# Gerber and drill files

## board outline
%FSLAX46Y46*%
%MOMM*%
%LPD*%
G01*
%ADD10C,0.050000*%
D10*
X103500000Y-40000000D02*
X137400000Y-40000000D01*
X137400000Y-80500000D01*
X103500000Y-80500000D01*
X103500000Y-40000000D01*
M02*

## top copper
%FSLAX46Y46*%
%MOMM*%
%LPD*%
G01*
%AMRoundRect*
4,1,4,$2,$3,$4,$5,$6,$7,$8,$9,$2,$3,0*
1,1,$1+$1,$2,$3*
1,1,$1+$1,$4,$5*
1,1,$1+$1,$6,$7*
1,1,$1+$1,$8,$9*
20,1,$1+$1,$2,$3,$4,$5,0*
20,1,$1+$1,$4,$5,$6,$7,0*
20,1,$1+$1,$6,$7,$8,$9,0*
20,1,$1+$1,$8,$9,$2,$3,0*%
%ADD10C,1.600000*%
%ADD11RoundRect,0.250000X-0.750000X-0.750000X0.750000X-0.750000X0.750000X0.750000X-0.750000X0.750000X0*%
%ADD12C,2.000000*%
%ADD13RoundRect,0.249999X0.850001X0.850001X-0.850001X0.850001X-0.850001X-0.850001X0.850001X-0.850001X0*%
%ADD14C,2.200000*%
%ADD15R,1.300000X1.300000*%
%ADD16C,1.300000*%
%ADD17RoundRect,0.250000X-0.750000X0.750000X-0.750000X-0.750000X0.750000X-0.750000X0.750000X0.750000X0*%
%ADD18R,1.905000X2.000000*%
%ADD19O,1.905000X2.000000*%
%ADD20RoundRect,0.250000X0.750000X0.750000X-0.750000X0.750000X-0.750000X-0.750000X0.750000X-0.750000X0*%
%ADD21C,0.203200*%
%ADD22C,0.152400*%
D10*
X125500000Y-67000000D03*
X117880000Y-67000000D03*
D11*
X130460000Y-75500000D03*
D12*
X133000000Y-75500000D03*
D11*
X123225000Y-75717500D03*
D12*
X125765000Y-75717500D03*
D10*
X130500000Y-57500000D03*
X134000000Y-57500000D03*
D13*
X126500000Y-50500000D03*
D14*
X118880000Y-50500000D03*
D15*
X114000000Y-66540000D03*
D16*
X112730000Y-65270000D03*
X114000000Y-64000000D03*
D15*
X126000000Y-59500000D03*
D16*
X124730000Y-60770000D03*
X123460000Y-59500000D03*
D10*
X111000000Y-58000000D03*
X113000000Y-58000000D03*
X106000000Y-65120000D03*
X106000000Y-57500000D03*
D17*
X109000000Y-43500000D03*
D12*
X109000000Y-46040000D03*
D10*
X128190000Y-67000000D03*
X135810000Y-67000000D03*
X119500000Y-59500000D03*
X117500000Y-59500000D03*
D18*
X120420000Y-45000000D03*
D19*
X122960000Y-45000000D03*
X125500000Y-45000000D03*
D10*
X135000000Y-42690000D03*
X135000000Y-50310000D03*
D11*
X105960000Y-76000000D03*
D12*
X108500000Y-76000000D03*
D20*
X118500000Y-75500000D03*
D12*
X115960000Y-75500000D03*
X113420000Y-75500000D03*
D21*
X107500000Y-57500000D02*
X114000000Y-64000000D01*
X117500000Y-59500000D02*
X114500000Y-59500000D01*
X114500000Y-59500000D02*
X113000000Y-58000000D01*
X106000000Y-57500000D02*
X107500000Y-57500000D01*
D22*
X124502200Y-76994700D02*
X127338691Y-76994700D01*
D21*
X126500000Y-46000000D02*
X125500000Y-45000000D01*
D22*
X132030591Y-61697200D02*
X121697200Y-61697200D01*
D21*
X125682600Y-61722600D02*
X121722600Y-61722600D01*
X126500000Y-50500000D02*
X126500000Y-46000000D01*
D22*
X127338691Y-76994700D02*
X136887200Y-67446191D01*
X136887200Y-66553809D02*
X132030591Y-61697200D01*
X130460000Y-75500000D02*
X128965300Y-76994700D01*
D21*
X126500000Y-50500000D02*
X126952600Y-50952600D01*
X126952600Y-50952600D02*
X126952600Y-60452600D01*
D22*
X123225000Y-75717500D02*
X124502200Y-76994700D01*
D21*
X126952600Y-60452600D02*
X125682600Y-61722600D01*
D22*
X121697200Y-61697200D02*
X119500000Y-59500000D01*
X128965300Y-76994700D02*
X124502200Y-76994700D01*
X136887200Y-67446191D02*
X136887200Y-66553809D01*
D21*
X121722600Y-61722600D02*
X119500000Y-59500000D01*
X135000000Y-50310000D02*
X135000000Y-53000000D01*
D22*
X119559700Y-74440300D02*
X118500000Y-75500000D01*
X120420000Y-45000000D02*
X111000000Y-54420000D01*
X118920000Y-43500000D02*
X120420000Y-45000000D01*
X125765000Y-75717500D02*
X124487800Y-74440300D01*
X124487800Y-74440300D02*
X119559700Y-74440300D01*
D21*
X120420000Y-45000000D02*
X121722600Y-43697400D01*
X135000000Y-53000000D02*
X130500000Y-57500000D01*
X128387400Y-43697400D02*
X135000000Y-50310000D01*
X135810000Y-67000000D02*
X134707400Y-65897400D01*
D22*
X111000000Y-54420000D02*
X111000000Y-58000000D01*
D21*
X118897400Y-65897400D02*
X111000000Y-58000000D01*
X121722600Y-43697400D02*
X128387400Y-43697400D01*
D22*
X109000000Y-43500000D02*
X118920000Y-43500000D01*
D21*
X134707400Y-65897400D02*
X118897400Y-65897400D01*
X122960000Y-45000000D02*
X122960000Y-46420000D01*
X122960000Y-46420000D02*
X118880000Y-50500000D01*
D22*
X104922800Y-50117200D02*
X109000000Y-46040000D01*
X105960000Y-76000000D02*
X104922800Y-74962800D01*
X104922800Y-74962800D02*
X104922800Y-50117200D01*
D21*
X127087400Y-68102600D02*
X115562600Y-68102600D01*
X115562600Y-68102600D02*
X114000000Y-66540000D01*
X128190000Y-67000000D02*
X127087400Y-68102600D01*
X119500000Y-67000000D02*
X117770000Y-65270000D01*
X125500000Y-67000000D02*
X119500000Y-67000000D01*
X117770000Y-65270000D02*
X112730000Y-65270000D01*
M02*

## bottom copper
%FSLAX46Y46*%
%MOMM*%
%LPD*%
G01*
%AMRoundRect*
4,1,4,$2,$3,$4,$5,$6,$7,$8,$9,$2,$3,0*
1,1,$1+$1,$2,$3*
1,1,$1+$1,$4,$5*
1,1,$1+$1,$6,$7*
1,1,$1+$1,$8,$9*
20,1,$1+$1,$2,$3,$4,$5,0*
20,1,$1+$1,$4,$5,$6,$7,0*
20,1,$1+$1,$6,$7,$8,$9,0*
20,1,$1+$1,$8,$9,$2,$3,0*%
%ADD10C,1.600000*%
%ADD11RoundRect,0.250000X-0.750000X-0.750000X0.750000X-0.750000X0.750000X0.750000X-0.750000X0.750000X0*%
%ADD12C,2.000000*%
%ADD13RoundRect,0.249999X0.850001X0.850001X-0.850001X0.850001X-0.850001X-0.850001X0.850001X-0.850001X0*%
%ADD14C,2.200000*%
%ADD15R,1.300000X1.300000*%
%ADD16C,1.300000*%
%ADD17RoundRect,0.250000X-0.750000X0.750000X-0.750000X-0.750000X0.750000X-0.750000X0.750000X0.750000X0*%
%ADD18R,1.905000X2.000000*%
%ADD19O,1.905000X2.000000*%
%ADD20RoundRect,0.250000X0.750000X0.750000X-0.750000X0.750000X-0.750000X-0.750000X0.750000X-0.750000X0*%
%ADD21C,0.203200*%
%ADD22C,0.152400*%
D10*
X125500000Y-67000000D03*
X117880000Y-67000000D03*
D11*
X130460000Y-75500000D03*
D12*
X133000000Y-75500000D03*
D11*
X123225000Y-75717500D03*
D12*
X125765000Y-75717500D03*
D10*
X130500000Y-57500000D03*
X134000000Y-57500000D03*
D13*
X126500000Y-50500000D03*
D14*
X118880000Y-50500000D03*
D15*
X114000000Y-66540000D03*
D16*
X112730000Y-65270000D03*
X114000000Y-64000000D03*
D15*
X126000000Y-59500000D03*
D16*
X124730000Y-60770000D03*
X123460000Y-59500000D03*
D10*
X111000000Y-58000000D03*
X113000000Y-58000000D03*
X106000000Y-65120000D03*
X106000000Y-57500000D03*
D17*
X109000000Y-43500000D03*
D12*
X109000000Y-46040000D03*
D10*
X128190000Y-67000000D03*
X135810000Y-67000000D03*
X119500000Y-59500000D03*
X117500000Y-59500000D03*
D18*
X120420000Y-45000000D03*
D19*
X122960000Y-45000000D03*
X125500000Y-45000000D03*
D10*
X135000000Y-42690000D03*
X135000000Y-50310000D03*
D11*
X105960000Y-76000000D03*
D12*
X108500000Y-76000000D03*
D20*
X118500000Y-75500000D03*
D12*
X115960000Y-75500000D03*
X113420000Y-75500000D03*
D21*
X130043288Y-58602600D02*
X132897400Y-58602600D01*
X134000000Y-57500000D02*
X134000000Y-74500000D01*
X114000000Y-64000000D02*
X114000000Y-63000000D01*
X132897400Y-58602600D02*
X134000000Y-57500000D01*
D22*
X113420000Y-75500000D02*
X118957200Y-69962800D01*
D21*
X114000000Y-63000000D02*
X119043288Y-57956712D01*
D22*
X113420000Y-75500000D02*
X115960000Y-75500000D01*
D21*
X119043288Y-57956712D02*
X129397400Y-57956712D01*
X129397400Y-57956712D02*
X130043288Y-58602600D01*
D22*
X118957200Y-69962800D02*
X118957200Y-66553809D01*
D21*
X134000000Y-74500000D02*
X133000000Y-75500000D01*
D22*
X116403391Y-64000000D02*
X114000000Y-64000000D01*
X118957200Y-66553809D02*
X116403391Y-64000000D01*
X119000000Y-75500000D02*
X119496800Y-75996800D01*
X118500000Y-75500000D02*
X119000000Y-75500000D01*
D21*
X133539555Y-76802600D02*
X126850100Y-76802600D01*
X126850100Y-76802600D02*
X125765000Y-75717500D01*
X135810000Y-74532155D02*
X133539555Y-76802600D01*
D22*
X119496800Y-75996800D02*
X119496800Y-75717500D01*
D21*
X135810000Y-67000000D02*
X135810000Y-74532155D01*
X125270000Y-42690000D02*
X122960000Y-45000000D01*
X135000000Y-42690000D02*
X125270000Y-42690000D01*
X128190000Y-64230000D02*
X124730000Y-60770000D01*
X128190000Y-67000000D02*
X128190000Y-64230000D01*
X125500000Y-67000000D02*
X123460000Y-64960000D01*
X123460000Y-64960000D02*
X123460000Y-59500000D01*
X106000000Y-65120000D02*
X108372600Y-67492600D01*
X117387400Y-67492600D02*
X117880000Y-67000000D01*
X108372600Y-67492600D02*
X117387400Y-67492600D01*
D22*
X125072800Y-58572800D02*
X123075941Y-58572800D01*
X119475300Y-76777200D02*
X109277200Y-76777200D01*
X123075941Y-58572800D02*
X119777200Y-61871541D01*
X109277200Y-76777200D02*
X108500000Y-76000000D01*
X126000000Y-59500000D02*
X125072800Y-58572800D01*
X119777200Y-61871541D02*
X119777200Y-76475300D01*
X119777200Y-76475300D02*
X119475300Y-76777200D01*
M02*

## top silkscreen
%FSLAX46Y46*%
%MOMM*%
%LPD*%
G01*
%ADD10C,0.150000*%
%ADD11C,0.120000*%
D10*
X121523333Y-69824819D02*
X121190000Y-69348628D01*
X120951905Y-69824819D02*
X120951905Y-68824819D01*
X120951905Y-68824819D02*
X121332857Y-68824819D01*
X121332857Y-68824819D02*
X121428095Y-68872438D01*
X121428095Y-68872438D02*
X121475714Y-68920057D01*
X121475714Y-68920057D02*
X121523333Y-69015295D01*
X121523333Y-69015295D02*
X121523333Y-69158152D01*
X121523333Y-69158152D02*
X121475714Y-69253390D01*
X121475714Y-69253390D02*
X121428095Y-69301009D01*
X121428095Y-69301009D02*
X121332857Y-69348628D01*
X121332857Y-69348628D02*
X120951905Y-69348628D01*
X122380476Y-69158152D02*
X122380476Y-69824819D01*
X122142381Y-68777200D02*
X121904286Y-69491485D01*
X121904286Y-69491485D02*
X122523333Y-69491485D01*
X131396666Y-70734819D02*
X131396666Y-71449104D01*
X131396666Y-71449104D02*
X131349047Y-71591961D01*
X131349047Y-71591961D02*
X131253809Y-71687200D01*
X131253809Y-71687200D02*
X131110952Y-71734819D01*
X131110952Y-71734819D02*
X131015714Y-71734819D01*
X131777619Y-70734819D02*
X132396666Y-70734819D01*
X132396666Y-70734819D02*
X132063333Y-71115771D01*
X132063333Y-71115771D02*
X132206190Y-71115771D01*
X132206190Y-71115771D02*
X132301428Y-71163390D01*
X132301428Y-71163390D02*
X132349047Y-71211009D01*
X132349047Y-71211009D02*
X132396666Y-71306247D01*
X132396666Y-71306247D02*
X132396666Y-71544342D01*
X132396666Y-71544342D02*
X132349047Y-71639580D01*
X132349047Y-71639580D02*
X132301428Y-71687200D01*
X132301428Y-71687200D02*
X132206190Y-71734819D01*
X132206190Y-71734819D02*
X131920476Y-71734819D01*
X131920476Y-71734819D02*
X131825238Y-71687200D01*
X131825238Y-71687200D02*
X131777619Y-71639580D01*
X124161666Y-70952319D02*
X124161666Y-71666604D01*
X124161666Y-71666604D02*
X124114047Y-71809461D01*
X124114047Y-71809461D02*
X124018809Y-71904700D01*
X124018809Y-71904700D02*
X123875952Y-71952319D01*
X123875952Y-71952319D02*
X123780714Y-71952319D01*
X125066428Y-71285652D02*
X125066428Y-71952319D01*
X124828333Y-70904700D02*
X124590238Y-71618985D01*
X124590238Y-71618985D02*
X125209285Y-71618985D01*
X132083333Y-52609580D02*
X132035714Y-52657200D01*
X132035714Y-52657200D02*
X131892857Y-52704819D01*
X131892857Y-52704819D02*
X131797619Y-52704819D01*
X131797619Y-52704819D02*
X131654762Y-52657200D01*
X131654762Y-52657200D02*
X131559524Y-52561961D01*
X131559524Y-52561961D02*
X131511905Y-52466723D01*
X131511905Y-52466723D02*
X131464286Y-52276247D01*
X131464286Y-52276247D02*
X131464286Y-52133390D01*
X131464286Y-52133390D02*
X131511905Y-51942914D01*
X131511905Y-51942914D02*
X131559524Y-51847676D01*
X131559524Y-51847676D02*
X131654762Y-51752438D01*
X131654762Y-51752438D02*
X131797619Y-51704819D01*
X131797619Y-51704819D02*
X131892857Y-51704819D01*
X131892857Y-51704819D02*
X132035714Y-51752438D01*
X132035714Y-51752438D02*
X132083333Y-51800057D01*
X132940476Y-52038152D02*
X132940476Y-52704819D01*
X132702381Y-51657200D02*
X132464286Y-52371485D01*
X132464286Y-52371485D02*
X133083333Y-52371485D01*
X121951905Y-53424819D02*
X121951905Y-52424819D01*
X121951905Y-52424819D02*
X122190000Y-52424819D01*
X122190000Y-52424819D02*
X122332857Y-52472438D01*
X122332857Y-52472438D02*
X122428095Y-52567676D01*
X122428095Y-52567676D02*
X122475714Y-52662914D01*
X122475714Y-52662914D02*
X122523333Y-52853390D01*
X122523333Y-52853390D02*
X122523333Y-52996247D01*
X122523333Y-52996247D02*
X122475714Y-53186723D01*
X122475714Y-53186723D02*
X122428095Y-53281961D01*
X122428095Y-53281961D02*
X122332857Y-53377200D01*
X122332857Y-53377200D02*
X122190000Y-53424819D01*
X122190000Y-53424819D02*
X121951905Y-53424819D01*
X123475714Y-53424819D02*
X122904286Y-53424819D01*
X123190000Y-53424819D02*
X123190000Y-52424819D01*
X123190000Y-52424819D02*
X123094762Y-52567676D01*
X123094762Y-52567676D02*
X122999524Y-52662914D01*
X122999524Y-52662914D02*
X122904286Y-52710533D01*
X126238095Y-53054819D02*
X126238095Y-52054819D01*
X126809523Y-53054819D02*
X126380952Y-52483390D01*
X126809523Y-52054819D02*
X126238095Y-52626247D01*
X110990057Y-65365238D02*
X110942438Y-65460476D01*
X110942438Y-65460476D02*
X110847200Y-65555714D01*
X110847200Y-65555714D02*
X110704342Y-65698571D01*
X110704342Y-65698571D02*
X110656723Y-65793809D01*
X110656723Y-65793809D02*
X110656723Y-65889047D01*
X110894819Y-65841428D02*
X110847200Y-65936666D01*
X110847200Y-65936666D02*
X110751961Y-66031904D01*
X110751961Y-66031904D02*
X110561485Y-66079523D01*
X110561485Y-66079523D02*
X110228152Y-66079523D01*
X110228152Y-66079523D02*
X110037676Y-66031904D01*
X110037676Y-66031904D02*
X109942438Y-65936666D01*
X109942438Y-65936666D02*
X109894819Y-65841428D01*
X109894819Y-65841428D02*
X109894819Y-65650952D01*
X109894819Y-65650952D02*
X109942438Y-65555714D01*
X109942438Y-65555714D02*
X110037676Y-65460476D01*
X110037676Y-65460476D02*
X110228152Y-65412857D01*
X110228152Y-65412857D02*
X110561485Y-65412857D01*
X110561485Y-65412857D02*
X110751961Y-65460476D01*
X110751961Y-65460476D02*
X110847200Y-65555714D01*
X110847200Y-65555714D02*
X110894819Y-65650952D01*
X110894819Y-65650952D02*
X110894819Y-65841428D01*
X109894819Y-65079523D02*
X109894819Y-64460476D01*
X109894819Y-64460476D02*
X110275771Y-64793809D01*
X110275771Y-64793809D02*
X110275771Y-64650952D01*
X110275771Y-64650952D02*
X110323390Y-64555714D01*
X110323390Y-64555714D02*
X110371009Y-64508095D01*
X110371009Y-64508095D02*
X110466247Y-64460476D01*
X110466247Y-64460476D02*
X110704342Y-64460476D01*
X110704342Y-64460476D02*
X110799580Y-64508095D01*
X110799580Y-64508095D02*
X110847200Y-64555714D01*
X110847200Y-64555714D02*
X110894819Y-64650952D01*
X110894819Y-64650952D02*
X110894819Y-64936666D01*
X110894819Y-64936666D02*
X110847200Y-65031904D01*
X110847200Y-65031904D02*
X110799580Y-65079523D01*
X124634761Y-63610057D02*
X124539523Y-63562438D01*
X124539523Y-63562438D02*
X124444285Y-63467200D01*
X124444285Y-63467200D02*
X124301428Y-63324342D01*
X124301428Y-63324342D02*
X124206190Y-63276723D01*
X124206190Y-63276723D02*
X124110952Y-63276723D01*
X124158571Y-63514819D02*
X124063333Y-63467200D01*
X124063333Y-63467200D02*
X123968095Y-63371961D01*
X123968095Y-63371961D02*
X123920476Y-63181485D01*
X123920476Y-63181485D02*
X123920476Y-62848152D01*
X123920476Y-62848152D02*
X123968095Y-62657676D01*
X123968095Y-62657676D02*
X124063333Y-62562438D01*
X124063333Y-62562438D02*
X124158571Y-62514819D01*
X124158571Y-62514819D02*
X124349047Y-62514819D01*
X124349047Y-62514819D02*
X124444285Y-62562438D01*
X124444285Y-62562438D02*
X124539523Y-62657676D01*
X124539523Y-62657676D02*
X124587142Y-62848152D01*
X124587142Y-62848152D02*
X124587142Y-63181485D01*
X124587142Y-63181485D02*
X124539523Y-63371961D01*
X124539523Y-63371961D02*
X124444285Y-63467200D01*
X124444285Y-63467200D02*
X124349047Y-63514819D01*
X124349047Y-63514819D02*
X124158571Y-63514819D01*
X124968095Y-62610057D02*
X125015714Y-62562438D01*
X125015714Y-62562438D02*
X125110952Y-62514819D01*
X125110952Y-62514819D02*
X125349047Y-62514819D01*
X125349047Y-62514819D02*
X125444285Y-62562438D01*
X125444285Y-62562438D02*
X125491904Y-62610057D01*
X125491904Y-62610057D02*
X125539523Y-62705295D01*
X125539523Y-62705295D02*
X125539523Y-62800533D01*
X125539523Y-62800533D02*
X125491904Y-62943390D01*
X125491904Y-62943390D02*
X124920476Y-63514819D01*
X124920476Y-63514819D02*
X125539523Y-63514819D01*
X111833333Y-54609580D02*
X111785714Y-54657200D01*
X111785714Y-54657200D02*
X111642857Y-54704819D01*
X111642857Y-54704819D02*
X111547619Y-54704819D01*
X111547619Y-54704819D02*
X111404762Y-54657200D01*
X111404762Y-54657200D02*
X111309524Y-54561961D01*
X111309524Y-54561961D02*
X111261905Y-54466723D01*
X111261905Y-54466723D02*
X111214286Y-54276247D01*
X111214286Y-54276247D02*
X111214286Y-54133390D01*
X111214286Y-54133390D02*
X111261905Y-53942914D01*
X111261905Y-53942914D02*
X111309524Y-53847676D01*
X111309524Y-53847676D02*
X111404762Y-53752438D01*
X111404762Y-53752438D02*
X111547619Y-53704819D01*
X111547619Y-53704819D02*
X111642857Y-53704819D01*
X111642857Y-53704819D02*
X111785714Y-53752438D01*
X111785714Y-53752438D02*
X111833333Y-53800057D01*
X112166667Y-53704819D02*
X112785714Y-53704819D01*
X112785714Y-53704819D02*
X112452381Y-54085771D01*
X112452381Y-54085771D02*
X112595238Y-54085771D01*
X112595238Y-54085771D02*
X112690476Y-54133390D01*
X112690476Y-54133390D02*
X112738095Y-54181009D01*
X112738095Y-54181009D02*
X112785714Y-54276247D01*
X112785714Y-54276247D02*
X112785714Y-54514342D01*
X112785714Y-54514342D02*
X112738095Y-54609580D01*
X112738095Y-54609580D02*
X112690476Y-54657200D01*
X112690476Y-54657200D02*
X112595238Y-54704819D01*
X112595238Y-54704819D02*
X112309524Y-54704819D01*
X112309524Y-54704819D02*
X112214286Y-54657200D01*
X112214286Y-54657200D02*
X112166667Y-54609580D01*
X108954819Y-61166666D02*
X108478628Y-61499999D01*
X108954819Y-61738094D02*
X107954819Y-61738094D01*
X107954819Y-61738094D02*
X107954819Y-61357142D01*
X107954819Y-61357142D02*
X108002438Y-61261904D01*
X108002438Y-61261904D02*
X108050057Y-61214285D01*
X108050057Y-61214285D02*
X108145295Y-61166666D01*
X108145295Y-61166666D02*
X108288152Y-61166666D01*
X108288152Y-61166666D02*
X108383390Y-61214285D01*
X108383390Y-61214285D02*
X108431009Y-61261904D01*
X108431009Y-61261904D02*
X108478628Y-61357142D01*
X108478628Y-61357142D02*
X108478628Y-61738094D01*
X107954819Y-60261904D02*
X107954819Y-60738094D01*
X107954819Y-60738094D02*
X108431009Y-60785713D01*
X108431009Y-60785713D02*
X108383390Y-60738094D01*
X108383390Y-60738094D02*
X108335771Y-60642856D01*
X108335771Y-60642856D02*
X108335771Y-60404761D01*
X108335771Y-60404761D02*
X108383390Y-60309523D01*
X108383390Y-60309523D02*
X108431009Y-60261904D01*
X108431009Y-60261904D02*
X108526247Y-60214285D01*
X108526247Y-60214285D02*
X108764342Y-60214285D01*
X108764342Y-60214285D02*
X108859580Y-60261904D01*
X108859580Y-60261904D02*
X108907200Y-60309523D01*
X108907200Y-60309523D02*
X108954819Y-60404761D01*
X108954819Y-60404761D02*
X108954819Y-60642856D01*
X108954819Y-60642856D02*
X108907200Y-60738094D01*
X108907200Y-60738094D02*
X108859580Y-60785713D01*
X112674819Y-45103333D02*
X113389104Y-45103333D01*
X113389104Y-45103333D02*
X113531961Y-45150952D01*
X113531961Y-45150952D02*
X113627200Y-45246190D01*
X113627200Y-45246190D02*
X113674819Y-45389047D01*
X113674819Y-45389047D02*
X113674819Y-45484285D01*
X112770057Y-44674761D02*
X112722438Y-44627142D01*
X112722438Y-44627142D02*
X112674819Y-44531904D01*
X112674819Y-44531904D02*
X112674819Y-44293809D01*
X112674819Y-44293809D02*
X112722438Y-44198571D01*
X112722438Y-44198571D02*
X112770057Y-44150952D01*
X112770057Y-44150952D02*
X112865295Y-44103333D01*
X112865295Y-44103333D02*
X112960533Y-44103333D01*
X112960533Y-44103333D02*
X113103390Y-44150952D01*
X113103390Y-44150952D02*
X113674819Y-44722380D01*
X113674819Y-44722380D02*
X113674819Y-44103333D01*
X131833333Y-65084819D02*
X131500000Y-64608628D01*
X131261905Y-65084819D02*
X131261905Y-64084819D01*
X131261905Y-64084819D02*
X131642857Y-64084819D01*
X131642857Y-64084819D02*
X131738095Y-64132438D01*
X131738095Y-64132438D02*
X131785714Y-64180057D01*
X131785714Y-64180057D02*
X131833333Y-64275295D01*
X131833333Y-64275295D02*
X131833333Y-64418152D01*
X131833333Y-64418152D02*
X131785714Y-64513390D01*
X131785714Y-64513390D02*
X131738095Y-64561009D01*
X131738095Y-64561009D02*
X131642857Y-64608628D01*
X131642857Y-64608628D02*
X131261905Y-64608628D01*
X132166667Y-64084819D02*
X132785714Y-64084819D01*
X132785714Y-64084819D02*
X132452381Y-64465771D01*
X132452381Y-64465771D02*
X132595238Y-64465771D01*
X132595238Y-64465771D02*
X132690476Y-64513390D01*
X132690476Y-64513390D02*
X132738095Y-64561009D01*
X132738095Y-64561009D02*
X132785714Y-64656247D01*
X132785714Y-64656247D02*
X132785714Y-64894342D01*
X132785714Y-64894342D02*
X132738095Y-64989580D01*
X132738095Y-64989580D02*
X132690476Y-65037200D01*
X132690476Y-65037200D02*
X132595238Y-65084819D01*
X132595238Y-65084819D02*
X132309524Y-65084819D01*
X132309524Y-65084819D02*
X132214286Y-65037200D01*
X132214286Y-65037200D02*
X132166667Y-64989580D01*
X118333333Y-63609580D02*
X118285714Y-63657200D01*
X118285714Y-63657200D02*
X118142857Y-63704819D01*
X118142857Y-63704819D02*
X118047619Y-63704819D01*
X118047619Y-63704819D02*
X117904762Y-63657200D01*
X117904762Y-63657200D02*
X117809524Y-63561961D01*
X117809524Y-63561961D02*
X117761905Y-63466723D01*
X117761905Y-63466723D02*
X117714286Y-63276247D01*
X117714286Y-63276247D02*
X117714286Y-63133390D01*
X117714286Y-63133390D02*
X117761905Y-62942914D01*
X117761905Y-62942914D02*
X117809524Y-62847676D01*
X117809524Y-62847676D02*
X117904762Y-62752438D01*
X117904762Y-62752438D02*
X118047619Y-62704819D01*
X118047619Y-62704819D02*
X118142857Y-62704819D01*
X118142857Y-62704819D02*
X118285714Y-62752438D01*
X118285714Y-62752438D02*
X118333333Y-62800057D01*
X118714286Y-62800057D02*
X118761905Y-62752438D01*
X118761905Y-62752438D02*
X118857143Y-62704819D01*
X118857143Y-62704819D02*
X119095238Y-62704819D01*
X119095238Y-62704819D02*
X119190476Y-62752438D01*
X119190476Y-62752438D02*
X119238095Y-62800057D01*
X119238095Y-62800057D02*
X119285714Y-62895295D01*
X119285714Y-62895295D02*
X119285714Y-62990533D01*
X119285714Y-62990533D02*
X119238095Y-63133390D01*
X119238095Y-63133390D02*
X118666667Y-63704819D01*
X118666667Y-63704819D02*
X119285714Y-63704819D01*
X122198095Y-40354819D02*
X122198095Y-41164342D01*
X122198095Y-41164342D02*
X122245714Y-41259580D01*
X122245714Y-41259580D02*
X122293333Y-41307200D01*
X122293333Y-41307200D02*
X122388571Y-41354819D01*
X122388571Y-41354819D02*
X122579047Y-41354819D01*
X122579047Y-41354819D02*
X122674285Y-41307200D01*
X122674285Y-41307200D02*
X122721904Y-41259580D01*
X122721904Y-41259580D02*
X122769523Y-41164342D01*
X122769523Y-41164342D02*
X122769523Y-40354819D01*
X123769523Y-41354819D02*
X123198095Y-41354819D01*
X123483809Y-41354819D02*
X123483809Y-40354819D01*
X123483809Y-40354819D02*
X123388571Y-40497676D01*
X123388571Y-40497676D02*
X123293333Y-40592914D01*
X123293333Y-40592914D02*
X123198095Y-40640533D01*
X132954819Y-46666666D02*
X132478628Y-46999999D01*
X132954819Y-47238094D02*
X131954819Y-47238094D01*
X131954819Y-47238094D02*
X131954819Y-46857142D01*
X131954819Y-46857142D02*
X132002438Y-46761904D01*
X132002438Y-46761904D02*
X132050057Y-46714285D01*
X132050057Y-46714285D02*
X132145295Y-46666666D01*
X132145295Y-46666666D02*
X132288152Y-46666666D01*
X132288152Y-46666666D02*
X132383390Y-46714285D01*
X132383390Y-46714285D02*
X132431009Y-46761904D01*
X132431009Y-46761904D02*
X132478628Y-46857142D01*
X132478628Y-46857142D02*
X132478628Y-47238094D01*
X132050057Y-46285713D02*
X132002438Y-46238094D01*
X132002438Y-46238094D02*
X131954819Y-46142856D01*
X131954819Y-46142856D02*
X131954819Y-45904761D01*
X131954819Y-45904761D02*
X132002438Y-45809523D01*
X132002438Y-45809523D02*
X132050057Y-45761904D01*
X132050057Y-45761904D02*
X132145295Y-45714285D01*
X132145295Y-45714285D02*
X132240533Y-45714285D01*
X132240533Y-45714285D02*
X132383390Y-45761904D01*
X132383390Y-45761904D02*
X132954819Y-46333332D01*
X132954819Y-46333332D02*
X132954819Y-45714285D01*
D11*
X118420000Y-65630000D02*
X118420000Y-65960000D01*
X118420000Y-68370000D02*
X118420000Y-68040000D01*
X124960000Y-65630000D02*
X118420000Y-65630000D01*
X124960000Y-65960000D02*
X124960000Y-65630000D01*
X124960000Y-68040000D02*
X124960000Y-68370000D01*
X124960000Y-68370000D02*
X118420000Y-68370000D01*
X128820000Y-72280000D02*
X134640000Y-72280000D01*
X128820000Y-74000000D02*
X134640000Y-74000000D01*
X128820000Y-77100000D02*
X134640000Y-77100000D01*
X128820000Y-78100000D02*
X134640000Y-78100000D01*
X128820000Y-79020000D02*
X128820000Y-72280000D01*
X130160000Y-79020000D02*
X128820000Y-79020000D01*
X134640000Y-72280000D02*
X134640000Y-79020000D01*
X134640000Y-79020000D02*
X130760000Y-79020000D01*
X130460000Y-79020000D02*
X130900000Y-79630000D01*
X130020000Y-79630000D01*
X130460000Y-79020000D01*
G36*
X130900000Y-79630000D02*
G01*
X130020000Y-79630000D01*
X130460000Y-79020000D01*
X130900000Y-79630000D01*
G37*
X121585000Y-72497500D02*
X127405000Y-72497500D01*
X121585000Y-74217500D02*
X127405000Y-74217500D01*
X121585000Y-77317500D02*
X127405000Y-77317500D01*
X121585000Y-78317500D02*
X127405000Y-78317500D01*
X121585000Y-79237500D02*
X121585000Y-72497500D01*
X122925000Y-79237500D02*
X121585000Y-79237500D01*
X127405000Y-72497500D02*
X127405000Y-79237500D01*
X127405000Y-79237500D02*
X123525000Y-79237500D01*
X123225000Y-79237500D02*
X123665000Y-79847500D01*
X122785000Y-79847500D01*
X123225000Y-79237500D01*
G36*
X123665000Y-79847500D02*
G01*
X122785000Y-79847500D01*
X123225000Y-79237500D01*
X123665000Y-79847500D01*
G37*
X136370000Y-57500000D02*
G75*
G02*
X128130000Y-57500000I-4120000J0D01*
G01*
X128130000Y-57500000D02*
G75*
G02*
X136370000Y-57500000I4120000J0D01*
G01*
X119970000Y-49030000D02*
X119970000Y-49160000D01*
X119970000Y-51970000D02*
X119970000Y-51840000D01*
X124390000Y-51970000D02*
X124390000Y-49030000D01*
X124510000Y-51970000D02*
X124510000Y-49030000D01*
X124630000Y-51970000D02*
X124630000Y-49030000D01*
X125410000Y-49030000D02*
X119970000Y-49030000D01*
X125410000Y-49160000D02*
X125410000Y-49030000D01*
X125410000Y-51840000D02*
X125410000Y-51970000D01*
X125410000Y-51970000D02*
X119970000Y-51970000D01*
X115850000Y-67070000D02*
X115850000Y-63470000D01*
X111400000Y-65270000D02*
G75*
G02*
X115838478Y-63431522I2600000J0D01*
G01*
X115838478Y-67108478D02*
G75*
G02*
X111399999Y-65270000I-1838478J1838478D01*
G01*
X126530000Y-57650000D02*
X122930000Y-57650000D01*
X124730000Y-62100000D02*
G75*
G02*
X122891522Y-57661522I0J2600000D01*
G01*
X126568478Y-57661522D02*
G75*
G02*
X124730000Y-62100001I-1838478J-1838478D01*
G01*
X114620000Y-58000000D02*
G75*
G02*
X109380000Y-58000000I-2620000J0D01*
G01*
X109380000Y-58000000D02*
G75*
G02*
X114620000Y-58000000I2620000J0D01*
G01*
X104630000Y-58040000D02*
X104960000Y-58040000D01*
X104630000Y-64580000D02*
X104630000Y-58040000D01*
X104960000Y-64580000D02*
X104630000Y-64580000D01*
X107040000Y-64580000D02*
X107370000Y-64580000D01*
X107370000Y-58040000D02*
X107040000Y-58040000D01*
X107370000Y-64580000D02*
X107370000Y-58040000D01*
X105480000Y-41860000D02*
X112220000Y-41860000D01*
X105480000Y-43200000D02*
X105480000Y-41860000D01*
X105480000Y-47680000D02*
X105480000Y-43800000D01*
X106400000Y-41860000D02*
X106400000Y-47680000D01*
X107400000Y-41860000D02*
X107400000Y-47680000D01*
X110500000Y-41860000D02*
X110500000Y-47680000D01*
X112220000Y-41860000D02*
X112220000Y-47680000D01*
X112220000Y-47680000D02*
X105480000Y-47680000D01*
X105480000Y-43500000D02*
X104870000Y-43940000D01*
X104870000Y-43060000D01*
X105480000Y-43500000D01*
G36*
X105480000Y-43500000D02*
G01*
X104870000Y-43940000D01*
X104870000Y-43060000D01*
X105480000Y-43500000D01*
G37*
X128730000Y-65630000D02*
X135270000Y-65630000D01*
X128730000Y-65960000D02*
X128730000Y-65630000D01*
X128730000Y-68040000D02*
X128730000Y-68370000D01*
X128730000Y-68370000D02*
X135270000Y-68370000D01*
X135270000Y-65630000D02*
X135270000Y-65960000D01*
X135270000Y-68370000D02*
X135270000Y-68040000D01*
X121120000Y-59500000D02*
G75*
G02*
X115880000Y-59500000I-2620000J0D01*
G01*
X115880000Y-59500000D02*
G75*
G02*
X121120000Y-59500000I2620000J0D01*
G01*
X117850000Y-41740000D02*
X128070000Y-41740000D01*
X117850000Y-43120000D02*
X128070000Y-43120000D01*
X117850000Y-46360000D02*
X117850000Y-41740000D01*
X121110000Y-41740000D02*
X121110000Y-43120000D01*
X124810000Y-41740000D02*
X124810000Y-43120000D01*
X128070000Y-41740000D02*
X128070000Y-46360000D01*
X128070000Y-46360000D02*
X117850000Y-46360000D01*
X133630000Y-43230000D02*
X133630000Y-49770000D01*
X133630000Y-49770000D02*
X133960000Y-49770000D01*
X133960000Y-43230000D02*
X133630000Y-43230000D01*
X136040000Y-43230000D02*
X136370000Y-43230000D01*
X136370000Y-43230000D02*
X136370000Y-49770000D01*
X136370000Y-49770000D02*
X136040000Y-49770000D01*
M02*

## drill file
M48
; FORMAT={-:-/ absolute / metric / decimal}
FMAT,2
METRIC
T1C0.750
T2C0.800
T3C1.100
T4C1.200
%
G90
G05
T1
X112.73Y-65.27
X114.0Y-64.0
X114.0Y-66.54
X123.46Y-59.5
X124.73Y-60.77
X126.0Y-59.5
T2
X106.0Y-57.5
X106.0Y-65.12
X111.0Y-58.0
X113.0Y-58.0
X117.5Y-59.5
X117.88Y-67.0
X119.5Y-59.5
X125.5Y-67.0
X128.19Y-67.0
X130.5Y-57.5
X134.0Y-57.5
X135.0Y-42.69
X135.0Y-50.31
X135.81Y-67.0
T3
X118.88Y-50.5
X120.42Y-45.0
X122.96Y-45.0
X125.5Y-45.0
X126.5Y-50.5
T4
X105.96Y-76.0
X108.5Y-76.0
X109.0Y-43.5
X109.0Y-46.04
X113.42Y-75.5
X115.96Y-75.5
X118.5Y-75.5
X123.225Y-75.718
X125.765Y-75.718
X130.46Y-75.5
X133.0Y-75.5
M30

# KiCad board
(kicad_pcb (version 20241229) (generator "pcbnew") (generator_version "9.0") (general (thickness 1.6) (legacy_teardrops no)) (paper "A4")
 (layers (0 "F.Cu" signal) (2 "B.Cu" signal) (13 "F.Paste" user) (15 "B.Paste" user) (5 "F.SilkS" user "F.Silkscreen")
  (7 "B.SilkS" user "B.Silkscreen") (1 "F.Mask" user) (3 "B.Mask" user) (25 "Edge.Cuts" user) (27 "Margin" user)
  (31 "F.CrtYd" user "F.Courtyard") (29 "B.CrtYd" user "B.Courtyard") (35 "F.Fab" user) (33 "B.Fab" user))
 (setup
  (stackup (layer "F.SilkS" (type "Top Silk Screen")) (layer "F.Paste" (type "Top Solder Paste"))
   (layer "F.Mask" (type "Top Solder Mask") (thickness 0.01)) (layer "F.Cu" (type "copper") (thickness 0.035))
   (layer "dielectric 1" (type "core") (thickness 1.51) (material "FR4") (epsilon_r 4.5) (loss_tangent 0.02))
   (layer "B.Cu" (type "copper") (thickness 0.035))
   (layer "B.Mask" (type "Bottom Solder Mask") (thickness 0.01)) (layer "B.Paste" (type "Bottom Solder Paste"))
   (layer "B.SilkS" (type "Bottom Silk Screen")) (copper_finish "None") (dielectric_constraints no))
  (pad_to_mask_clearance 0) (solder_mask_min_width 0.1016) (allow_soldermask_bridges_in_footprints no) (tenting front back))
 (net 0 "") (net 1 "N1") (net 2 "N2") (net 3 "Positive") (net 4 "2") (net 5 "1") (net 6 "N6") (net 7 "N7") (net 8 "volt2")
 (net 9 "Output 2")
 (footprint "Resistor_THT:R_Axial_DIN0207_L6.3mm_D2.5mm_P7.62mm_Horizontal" (layer "F.Cu") (at 125.5 67 180)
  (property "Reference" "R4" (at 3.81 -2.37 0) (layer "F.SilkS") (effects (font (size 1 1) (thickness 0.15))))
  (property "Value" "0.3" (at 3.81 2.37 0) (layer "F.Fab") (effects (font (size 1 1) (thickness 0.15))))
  (fp_line (start 7.08 1.37) (end 7.08 1.04) (stroke (width 0.12) (type solid)) (layer "F.SilkS"))
  (fp_line (start 7.08 -1.37) (end 7.08 -1.04) (stroke (width 0.12) (type solid)) (layer "F.SilkS"))
  (fp_line (start 0.54 1.37) (end 7.08 1.37) (stroke (width 0.12) (type solid)) (layer "F.SilkS"))
  (fp_line (start 0.54 1.04) (end 0.54 1.37) (stroke (width 0.12) (type solid)) (layer "F.SilkS"))
  (fp_line (start 0.54 -1.04) (end 0.54 -1.37) (stroke (width 0.12) (type solid)) (layer "F.SilkS"))
  (fp_line (start 0.54 -1.37) (end 7.08 -1.37) (stroke (width 0.12) (type solid)) (layer "F.SilkS"))
  (pad "1" thru_hole circle (at 0 0 180) (size 1.6 1.6) (drill 0.8) (layers "*.Cu" "*.Mask") (remove_unused_layers no) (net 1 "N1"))
  (pad "2" thru_hole circle (at 7.62 0 180) (size 1.6 1.6) (drill 0.8) (layers "*.Cu" "*.Mask") (remove_unused_layers no) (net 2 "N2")))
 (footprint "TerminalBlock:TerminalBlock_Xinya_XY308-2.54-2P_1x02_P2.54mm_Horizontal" (layer "F.Cu") (at 130.46 75.5)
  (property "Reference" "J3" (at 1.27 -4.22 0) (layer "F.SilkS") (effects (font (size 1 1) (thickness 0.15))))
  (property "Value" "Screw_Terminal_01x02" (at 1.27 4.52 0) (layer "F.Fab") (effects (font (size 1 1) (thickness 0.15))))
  (fp_line (start -1.64 -3.22) (end 4.18 -3.22) (stroke (width 0.12) (type solid)) (layer "F.SilkS"))
  (fp_line (start -1.64 -1.5) (end 4.18 -1.5) (stroke (width 0.12) (type solid)) (layer "F.SilkS"))
  (fp_line (start -1.64 1.6) (end 4.18 1.6) (stroke (width 0.12) (type solid)) (layer "F.SilkS"))
  (fp_line (start -1.64 2.6) (end 4.18 2.6) (stroke (width 0.12) (type solid)) (layer "F.SilkS"))
  (fp_line (start -1.64 3.52) (end -1.64 -3.22) (stroke (width 0.12) (type solid)) (layer "F.SilkS"))
  (fp_line (start -0.3 3.52) (end -1.64 3.52) (stroke (width 0.12) (type solid)) (layer "F.SilkS"))
  (fp_line (start 4.18 -3.22) (end 4.18 3.52) (stroke (width 0.12) (type solid)) (layer "F.SilkS"))
  (fp_line (start 4.18 3.52) (end 0.3 3.52) (stroke (width 0.12) (type solid)) (layer "F.SilkS"))
  (fp_poly (pts (xy 0 3.52) (xy 0.44 4.13) (xy -0.44 4.13)) (stroke (width 0.12) (type solid)) (fill yes) (layer "F.SilkS"))
  (pad "1" thru_hole roundrect (at 0 0) (size 2 2) (drill 1.2) (layers "*.Cu" "*.Mask") (remove_unused_layers no) (roundrect_rratio 0.125)
   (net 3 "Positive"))
  (pad "2" thru_hole circle (at 2.54 0) (size 2 2) (drill 1.2) (layers "*.Cu" "*.Mask") (remove_unused_layers no) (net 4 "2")))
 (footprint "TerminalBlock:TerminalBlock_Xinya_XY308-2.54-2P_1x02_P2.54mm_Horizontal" (layer "F.Cu") (at 123.225 75.7175)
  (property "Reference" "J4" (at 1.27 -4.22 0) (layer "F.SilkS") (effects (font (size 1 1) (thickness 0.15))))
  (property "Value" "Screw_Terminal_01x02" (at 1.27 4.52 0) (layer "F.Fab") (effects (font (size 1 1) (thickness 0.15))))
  (fp_line (start -1.64 -3.22) (end 4.18 -3.22) (stroke (width 0.12) (type solid)) (layer "F.SilkS"))
  (fp_line (start -1.64 -1.5) (end 4.18 -1.5) (stroke (width 0.12) (type solid)) (layer "F.SilkS"))
  (fp_line (start -1.64 1.6) (end 4.18 1.6) (stroke (width 0.12) (type solid)) (layer "F.SilkS"))
  (fp_line (start -1.64 2.6) (end 4.18 2.6) (stroke (width 0.12) (type solid)) (layer "F.SilkS"))
  (fp_line (start -1.64 3.52) (end -1.64 -3.22) (stroke (width 0.12) (type solid)) (layer "F.SilkS"))
  (fp_line (start -0.3 3.52) (end -1.64 3.52) (stroke (width 0.12) (type solid)) (layer "F.SilkS"))
  (fp_line (start 4.18 -3.22) (end 4.18 3.52) (stroke (width 0.12) (type solid)) (layer "F.SilkS"))
  (fp_line (start 4.18 3.52) (end 0.3 3.52) (stroke (width 0.12) (type solid)) (layer "F.SilkS"))
  (fp_poly (pts (xy 0 3.52) (xy 0.44 4.13) (xy -0.44 4.13)) (stroke (width 0.12) (type solid)) (fill yes) (layer "F.SilkS"))
  (pad "1" thru_hole roundrect (at 0 0) (size 2 2) (drill 1.2) (layers "*.Cu" "*.Mask") (remove_unused_layers no) (roundrect_rratio 0.125)
   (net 3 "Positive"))
  (pad "2" thru_hole circle (at 2.54 0) (size 2 2) (drill 1.2) (layers "*.Cu" "*.Mask") (remove_unused_layers no) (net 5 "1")))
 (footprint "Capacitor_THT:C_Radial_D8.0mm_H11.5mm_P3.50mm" (layer "F.Cu") (at 130.5 57.5)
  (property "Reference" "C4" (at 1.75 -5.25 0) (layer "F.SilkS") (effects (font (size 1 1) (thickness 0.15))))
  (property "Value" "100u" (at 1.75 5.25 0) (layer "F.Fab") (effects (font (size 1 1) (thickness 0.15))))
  (fp_circle (center 1.75 0) (end 5.87 0) (stroke (width 0.12) (type solid)) (fill no) (layer "F.SilkS"))
  (pad "1" thru_hole circle (at 0 0) (size 1.6 1.6) (drill 0.8) (layers "*.Cu" "*.Mask") (remove_unused_layers no) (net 5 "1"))
  (pad "2" thru_hole circle (at 3.5 0) (size 1.6 1.6) (drill 0.8) (layers "*.Cu" "*.Mask") (remove_unused_layers no) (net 4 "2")))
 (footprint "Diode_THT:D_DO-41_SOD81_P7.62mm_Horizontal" (layer "F.Cu") (at 126.5 50.5 180)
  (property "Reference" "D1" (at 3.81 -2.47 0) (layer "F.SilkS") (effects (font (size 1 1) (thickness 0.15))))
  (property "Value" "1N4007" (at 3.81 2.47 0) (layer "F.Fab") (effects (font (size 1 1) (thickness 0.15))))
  (fp_line (start 6.53 1.47) (end 6.53 1.34) (stroke (width 0.12) (type solid)) (layer "F.SilkS"))
  (fp_line (start 6.53 -1.47) (end 6.53 -1.34) (stroke (width 0.12) (type solid)) (layer "F.SilkS"))
  (fp_line (start 2.11 -1.47) (end 2.11 1.47) (stroke (width 0.12) (type solid)) (layer "F.SilkS"))
  (fp_line (start 1.99 -1.47) (end 1.99 1.47) (stroke (width 0.12) (type solid)) (layer "F.SilkS"))
  (fp_line (start 1.87 -1.47) (end 1.87 1.47) (stroke (width 0.12) (type solid)) (layer "F.SilkS"))
  (fp_line (start 1.09 1.47) (end 6.53 1.47) (stroke (width 0.12) (type solid)) (layer "F.SilkS"))
  (fp_line (start 1.09 1.34) (end 1.09 1.47) (stroke (width 0.12) (type solid)) (layer "F.SilkS"))
  (fp_line (start 1.09 -1.34) (end 1.09 -1.47) (stroke (width 0.12) (type solid)) (layer "F.SilkS"))
  (fp_line (start 1.09 -1.47) (end 6.53 -1.47) (stroke (width 0.12) (type solid)) (layer "F.SilkS"))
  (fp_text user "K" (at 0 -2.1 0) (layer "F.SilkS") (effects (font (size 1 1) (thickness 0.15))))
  (pad "1" thru_hole roundrect (at 0 0 180) (size 2.2 2.2) (drill 1.1) (layers "*.Cu" "*.Mask") (remove_unused_layers no)
   (roundrect_rratio 0.113636) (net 3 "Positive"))
  (pad "2" thru_hole circle (at 7.62 0 180) (size 2.2 2.2) (drill 1.1) (layers "*.Cu" "*.Mask") (remove_unused_layers no) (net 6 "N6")))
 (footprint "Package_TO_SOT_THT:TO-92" (layer "F.Cu") (at 114 66.54 90)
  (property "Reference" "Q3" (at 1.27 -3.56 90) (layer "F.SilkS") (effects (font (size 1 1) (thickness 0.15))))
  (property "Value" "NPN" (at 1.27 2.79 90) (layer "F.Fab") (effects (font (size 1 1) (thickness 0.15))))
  (fp_line (start -0.53 1.85) (end 3.07 1.85) (stroke (width 0.12) (type solid)) (layer "F.SilkS"))
  (fp_arc (start 1.27 -2.6) (mid 3.672087 -0.994977) (end 3.108478 1.838478) (stroke (width 0.12) (type solid)) (layer "F.SilkS"))
  (fp_arc (start -0.568478 1.838478) (mid -1.132087 -0.994977) (end 1.27 -2.6) (stroke (width 0.12) (type solid)) (layer "F.SilkS"))
  (pad "1" thru_hole rect (at 0 0 90) (size 1.3 1.3) (drill 0.75) (layers "*.Cu" "*.Mask") (remove_unused_layers no) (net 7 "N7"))
  (pad "2" thru_hole circle (at 1.27 -1.27 90) (size 1.3 1.3) (drill 0.75) (layers "*.Cu" "*.Mask") (remove_unused_layers no) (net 1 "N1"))
  (pad "3" thru_hole circle (at 2.54 0 90) (size 1.3 1.3) (drill 0.75) (layers "*.Cu" "*.Mask") (remove_unused_layers no) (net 4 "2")))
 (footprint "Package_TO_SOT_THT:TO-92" (layer "F.Cu") (at 126 59.5 180)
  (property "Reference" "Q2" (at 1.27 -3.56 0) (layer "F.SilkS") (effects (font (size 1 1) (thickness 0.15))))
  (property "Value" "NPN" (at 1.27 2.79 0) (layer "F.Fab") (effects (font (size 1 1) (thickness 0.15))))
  (fp_line (start -0.53 1.85) (end 3.07 1.85) (stroke (width 0.12) (type solid)) (layer "F.SilkS"))
  (fp_arc (start 1.27 -2.6) (mid 3.672087 -0.994977) (end 3.108478 1.838478) (stroke (width 0.12) (type solid)) (layer "F.SilkS"))
  (fp_arc (start -0.568478 1.838478) (mid -1.132087 -0.994977) (end 1.27 -2.6) (stroke (width 0.12) (type solid)) (layer "F.SilkS"))
  (pad "1" thru_hole rect (at 0 0 180) (size 1.3 1.3) (drill 0.75) (layers "*.Cu" "*.Mask") (remove_unused_layers no) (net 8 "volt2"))
  (pad "2" thru_hole circle (at 1.27 -1.27 180) (size 1.3 1.3) (drill 0.75) (layers "*.Cu" "*.Mask") (remove_unused_layers no) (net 7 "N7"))
  (pad "3" thru_hole circle (at 2.54 0 180) (size 1.3 1.3) (drill 0.75) (layers "*.Cu" "*.Mask") (remove_unused_layers no) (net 1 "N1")))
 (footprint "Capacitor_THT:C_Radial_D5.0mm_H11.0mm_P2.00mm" (layer "F.Cu") (at 111 58)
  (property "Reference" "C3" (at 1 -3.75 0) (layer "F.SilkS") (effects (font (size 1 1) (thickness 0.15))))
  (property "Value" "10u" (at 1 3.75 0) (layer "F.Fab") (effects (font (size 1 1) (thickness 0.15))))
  (fp_circle (center 1 0) (end 3.62 0) (stroke (width 0.12) (type solid)) (fill no) (layer "F.SilkS"))
  (pad "1" thru_hole circle (at 0 0) (size 1.6 1.6) (drill 0.8) (layers "*.Cu" "*.Mask") (remove_unused_layers no) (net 5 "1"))
  (pad "2" thru_hole circle (at 2 0) (size 1.6 1.6) (drill 0.8) (layers "*.Cu" "*.Mask") (remove_unused_layers no) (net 4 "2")))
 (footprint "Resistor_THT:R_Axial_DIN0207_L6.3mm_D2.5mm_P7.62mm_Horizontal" (layer "F.Cu") (at 106 65.12 90)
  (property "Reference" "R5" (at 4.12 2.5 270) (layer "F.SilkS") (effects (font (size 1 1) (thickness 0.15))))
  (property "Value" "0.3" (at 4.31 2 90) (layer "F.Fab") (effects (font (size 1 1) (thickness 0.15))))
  (fp_line (start 7.08 -1.37) (end 7.08 -1.04) (stroke (width 0.12) (type solid)) (layer "F.SilkS"))
  (fp_line (start 0.54 -1.37) (end 7.08 -1.37) (stroke (width 0.12) (type solid)) (layer "F.SilkS"))
  (fp_line (start 0.54 -1.04) (end 0.54 -1.37) (stroke (width 0.12) (type solid)) (layer "F.SilkS"))
  (fp_line (start 0.54 1.04) (end 0.54 1.37) (stroke (width 0.12) (type solid)) (layer "F.SilkS"))
  (fp_line (start 7.08 1.37) (end 7.08 1.04) (stroke (width 0.12) (type solid)) (layer "F.SilkS"))
  (fp_line (start 0.54 1.37) (end 7.08 1.37) (stroke (width 0.12) (type solid)) (layer "F.SilkS"))
  (pad "1" thru_hole circle (at 0 0 90) (size 1.6 1.6) (drill 0.8) (layers "*.Cu" "*.Mask") (remove_unused_layers no) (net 2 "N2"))
  (pad "2" thru_hole circle (at 7.62 0 90) (size 1.6 1.6) (drill 0.8) (layers "*.Cu" "*.Mask") (remove_unused_layers no) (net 4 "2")))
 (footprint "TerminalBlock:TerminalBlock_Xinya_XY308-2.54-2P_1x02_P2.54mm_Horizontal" (layer "F.Cu") (at 109 43.5 -90)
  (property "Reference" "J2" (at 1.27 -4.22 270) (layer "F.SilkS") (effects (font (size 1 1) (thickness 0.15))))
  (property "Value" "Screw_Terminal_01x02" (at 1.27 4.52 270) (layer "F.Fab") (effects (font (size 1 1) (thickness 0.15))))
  (fp_line (start -1.64 3.52) (end -1.64 -3.22) (stroke (width 0.12) (type solid)) (layer "F.SilkS"))
  (fp_line (start -0.3 3.52) (end -1.64 3.52) (stroke (width 0.12) (type solid)) (layer "F.SilkS"))
  (fp_line (start 4.18 3.52) (end 0.3 3.52) (stroke (width 0.12) (type solid)) (layer "F.SilkS"))
  (fp_line (start -1.64 2.6) (end 4.18 2.6) (stroke (width 0.12) (type solid)) (layer "F.SilkS"))
  (fp_line (start -1.64 1.6) (end 4.18 1.6) (stroke (width 0.12) (type solid)) (layer "F.SilkS"))
  (fp_line (start -1.64 -1.5) (end 4.18 -1.5) (stroke (width 0.12) (type solid)) (layer "F.SilkS"))
  (fp_line (start -1.64 -3.22) (end 4.18 -3.22) (stroke (width 0.12) (type solid)) (layer "F.SilkS"))
  (fp_line (start 4.18 -3.22) (end 4.18 3.52) (stroke (width 0.12) (type solid)) (layer "F.SilkS"))
  (fp_poly (pts (xy 0 3.52) (xy 0.44 4.13) (xy -0.44 4.13)) (stroke (width 0.12) (type solid)) (fill yes) (layer "F.SilkS"))
  (pad "1" thru_hole roundrect (at 0 0 270) (size 2 2) (drill 1.2) (layers "*.Cu" "*.Mask") (remove_unused_layers no)
   (roundrect_rratio 0.125) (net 5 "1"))
  (pad "2" thru_hole circle (at 2.54 0 270) (size 2 2) (drill 1.2) (layers "*.Cu" "*.Mask") (remove_unused_layers no) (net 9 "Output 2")))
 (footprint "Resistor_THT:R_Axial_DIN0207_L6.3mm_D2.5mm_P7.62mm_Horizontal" (layer "F.Cu") (at 128.19 67)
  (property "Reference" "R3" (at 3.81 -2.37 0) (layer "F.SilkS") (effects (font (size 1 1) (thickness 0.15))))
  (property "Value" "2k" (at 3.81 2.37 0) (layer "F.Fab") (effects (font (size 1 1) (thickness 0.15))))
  (fp_line (start 0.54 -1.37) (end 7.08 -1.37) (stroke (width 0.12) (type solid)) (layer "F.SilkS"))
  (fp_line (start 0.54 -1.04) (end 0.54 -1.37) (stroke (width 0.12) (type solid)) (layer "F.SilkS"))
  (fp_line (start 0.54 1.04) (end 0.54 1.37) (stroke (width 0.12) (type solid)) (layer "F.SilkS"))
  (fp_line (start 0.54 1.37) (end 7.08 1.37) (stroke (width 0.12) (type solid)) (layer "F.SilkS"))
  (fp_line (start 7.08 -1.37) (end 7.08 -1.04) (stroke (width 0.12) (type solid)) (layer "F.SilkS"))
  (fp_line (start 7.08 1.37) (end 7.08 1.04) (stroke (width 0.12) (type solid)) (layer "F.SilkS"))
  (pad "1" thru_hole circle (at 0 0) (size 1.6 1.6) (drill 0.8) (layers "*.Cu" "*.Mask") (remove_unused_layers no) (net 7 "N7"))
  (pad "2" thru_hole circle (at 7.62 0) (size 1.6 1.6) (drill 0.8) (layers "*.Cu" "*.Mask") (remove_unused_layers no) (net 5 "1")))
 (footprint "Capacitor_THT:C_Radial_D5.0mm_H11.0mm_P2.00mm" (layer "F.Cu") (at 119.5 59.5 180)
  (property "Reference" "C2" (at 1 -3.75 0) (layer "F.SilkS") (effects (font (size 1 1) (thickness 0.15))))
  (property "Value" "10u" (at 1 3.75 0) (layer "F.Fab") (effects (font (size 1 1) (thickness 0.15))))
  (fp_circle (center 1 0) (end 3.62 0) (stroke (width 0.12) (type solid)) (fill no) (layer "F.SilkS"))
  (pad "1" thru_hole circle (at 0 0 180) (size 1.6 1.6) (drill 0.8) (layers "*.Cu" "*.Mask") (remove_unused_layers no) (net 3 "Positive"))
  (pad "2" thru_hole circle (at 2 0 180) (size 1.6 1.6) (drill 0.8) (layers "*.Cu" "*.Mask") (remove_unused_layers no) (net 4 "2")))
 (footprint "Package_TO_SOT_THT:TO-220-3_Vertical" (layer "F.Cu") (at 120.42 45)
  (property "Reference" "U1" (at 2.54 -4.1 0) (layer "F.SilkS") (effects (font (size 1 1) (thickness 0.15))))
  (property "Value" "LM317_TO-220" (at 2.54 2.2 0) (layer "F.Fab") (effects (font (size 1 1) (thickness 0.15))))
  (fp_line (start -2.57 -3.26) (end 7.65 -3.26) (stroke (width 0.12) (type solid)) (layer "F.SilkS"))
  (fp_line (start -2.57 -1.88) (end 7.65 -1.88) (stroke (width 0.12) (type solid)) (layer "F.SilkS"))
  (fp_line (start -2.57 1.36) (end -2.57 -3.26) (stroke (width 0.12) (type solid)) (layer "F.SilkS"))
  (fp_line (start 0.69 -3.26) (end 0.69 -1.88) (stroke (width 0.12) (type solid)) (layer "F.SilkS"))
  (fp_line (start 4.39 -3.26) (end 4.39 -1.88) (stroke (width 0.12) (type solid)) (layer "F.SilkS"))
  (fp_line (start 7.65 -3.26) (end 7.65 1.36) (stroke (width 0.12) (type solid)) (layer "F.SilkS"))
  (fp_line (start 7.65 1.36) (end -2.57 1.36) (stroke (width 0.12) (type solid)) (layer "F.SilkS"))
  (pad "1" thru_hole rect (at 0 0) (size 1.905 2) (drill 1.1) (layers "*.Cu" "*.Mask") (remove_unused_layers no) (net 5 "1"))
  (pad "2" thru_hole oval (at 2.54 0) (size 1.905 2) (drill 1.1) (layers "*.Cu" "*.Mask") (remove_unused_layers no) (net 6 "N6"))
  (pad "3" thru_hole oval (at 5.08 0) (size 1.905 2) (drill 1.1) (layers "*.Cu" "*.Mask") (remove_unused_layers no) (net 3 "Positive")))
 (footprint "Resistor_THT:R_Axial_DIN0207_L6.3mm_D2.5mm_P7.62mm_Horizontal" (layer "F.Cu") (at 135 42.69 -90)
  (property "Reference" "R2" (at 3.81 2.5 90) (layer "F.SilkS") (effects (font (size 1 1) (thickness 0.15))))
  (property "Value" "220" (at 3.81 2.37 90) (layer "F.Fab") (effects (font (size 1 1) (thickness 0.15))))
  (fp_line (start 0.54 1.37) (end 7.08 1.37) (stroke (width 0.12) (type solid)) (layer "F.SilkS"))
  (fp_line (start 7.08 1.37) (end 7.08 1.04) (stroke (width 0.12) (type solid)) (layer "F.SilkS"))
  (fp_line (start 0.54 1.04) (end 0.54 1.37) (stroke (width 0.12) (type solid)) (layer "F.SilkS"))
  (fp_line (start 0.54 -1.04) (end 0.54 -1.37) (stroke (width 0.12) (type solid)) (layer "F.SilkS"))
  (fp_line (start 0.54 -1.37) (end 7.08 -1.37) (stroke (width 0.12) (type solid)) (layer "F.SilkS"))
  (fp_line (start 7.08 -1.37) (end 7.08 -1.04) (stroke (width 0.12) (type solid)) (layer "F.SilkS"))
  (pad "1" thru_hole circle (at 0 0 270) (size 1.6 1.6) (drill 0.8) (layers "*.Cu" "*.Mask") (remove_unused_layers no) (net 6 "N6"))
  (pad "2" thru_hole circle (at 7.62 0 270) (size 1.6 1.6) (drill 0.8) (layers "*.Cu" "*.Mask") (remove_unused_layers no) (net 5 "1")))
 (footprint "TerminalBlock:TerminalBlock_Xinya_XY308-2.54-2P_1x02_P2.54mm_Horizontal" (layer "B.Cu") (at 105.96 76)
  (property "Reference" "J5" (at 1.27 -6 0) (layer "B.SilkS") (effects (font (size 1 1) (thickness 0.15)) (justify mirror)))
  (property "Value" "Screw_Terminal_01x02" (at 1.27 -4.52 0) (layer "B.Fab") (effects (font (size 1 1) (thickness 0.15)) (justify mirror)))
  (pad "1" thru_hole roundrect (at 0 0) (size 2 2) (drill 1.2) (layers "*.Cu" "*.Mask") (remove_unused_layers no) (roundrect_rratio 0.125)
   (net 9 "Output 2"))
  (pad "2" thru_hole circle (at 2.54 0) (size 2 2) (drill 1.2) (layers "*.Cu" "*.Mask") (remove_unused_layers no) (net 8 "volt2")))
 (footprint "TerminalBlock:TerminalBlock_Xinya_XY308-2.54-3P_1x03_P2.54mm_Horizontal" (layer "B.Cu") (at 118.5 75.5 180)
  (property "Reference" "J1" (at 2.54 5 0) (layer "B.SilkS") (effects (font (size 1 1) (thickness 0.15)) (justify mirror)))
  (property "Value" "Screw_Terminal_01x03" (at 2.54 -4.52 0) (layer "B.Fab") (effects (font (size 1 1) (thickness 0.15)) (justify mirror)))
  (pad "1" thru_hole roundrect (at 0 0 180) (size 2 2) (drill 1.2) (layers "*.Cu" "*.Mask") (remove_unused_layers no)
   (roundrect_rratio 0.125) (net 5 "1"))
  (pad "2" thru_hole circle (at 2.54 0 180) (size 2 2) (drill 1.2) (layers "*.Cu" "*.Mask") (remove_unused_layers no) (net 4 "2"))
  (pad "3" thru_hole circle (at 5.08 0 180) (size 2 2) (drill 1.2) (layers "*.Cu" "*.Mask") (remove_unused_layers no) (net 4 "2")))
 (gr_rect (start 103.5 40) (end 137.4 80.5) (stroke (width 0.05) (type default)) (fill no) (layer "Edge.Cuts"))
 (segment (start 107.5 57.5) (end 114 64) (width 0.2032) (layer "F.Cu") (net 4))
 (segment (start 117.5 59.5) (end 114.5 59.5) (width 0.2032) (layer "F.Cu") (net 4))
 (segment (start 114.5 59.5) (end 113 58) (width 0.2032) (layer "F.Cu") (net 4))
 (segment (start 106 57.5) (end 107.5 57.5) (width 0.2032) (layer "F.Cu") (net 4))
 (segment (start 130.043288 58.6026) (end 132.8974 58.6026) (width 0.2032) (layer "B.Cu") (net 4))
 (segment (start 134 57.5) (end 134 74.5) (width 0.2032) (layer "B.Cu") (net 4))
 (segment (start 114 64) (end 114 63) (width 0.2032) (layer "B.Cu") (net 4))
 (segment (start 132.8974 58.6026) (end 134 57.5) (width 0.2032) (layer "B.Cu") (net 4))
 (segment (start 113.42 75.5) (end 118.9572 69.9628) (width 0.1524) (layer "B.Cu") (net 4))
 (segment (start 114 63) (end 119.043288 57.956712) (width 0.2032) (layer "B.Cu") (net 4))
 (segment (start 113.42 75.5) (end 115.96 75.5) (width 0.1524) (layer "B.Cu") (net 4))
 (segment (start 119.043288 57.956712) (end 129.3974 57.956712) (width 0.2032) (layer "B.Cu") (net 4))
 (segment (start 129.3974 57.956712) (end 130.043288 58.6026) (width 0.2032) (layer "B.Cu") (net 4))
 (segment (start 118.9572 69.9628) (end 118.9572 66.553809) (width 0.1524) (layer "B.Cu") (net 4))
 (segment (start 134 74.5) (end 133 75.5) (width 0.2032) (layer "B.Cu") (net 4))
 (segment (start 116.403391 64) (end 114 64) (width 0.1524) (layer "B.Cu") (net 4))
 (segment (start 118.9572 66.553809) (end 116.403391 64) (width 0.1524) (layer "B.Cu") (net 4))
 (segment (start 124.5022 76.9947) (end 127.338691 76.9947) (width 0.1524) (layer "F.Cu") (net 3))
 (segment (start 126.5 46) (end 125.5 45) (width 0.2032) (layer "F.Cu") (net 3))
 (segment (start 132.030591 61.6972) (end 121.6972 61.6972) (width 0.1524) (layer "F.Cu") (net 3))
 (segment (start 125.6826 61.7226) (end 121.7226 61.7226) (width 0.2032) (layer "F.Cu") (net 3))
 (segment (start 126.5 50.5) (end 126.5 46) (width 0.2032) (layer "F.Cu") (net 3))
 (segment (start 127.338691 76.9947) (end 136.8872 67.446191) (width 0.1524) (layer "F.Cu") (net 3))
 (segment (start 136.8872 66.553809) (end 132.030591 61.6972) (width 0.1524) (layer "F.Cu") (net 3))
 (segment (start 130.46 75.5) (end 128.9653 76.9947) (width 0.1524) (layer "F.Cu") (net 3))
 (segment (start 126.5 50.5) (end 126.9526 50.9526) (width 0.2032) (layer "F.Cu") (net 3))
 (segment (start 126.9526 50.9526) (end 126.9526 60.4526) (width 0.2032) (layer "F.Cu") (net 3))
 (segment (start 123.225 75.7175) (end 124.5022 76.9947) (width 0.1524) (layer "F.Cu") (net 3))
 (segment (start 126.9526 60.4526) (end 125.6826 61.7226) (width 0.2032) (layer "F.Cu") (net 3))
 (segment (start 121.6972 61.6972) (end 119.5 59.5) (width 0.1524) (layer "F.Cu") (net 3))
 (segment (start 128.9653 76.9947) (end 124.5022 76.9947) (width 0.1524) (layer "F.Cu") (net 3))
 (segment (start 136.8872 67.446191) (end 136.8872 66.553809) (width 0.1524) (layer "F.Cu") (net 3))
 (segment (start 121.7226 61.7226) (end 119.5 59.5) (width 0.2032) (layer "F.Cu") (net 3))
 (segment (start 135 50.31) (end 135 53) (width 0.2032) (layer "F.Cu") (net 5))
 (segment (start 119.5597 74.4403) (end 118.5 75.5) (width 0.1524) (layer "F.Cu") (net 5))
 (segment (start 120.42 45) (end 111 54.42) (width 0.1524) (layer "F.Cu") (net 5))
 (segment (start 118.92 43.5) (end 120.42 45) (width 0.1524) (layer "F.Cu") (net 5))
 (segment (start 125.765 75.7175) (end 124.4878 74.4403) (width 0.1524) (layer "F.Cu") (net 5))
 (segment (start 124.4878 74.4403) (end 119.5597 74.4403) (width 0.1524) (layer "F.Cu") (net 5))
 (segment (start 120.42 45) (end 121.7226 43.6974) (width 0.2032) (layer "F.Cu") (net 5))
 (segment (start 135 53) (end 130.5 57.5) (width 0.2032) (layer "F.Cu") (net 5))
 (segment (start 128.3874 43.6974) (end 135 50.31) (width 0.2032) (layer "F.Cu") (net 5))
 (segment (start 135.81 67) (end 134.7074 65.8974) (width 0.2032) (layer "F.Cu") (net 5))
 (segment (start 111 54.42) (end 111 58) (width 0.1524) (layer "F.Cu") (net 5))
 (segment (start 118.8974 65.8974) (end 111 58) (width 0.2032) (layer "F.Cu") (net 5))
 (segment (start 121.7226 43.6974) (end 128.3874 43.6974) (width 0.2032) (layer "F.Cu") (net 5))
 (segment (start 109 43.5) (end 118.92 43.5) (width 0.1524) (layer "F.Cu") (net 5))
 (segment (start 134.7074 65.8974) (end 118.8974 65.8974) (width 0.2032) (layer "F.Cu") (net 5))
 (segment (start 119 75.5) (end 119.4968 75.9968) (width 0.1524) (layer "B.Cu") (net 5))
 (segment (start 118.5 75.5) (end 119 75.5) (width 0.1524) (layer "B.Cu") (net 5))
 (segment (start 133.539555 76.8026) (end 126.8501 76.8026) (width 0.2032) (layer "B.Cu") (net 5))
 (segment (start 126.8501 76.8026) (end 125.765 75.7175) (width 0.2032) (layer "B.Cu") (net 5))
 (segment (start 135.81 74.532155) (end 133.539555 76.8026) (width 0.2032) (layer "B.Cu") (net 5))
 (segment (start 119.4968 75.9968) (end 119.4968 75.7175) (width 0.1524) (layer "B.Cu") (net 5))
 (segment (start 135.81 67) (end 135.81 74.532155) (width 0.2032) (layer "B.Cu") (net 5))
 (segment (start 122.96 45) (end 122.96 46.42) (width 0.2032) (layer "F.Cu") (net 6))
 (segment (start 122.96 46.42) (end 118.88 50.5) (width 0.2032) (layer "F.Cu") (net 6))
 (segment (start 125.27 42.69) (end 122.96 45) (width 0.2032) (layer "B.Cu") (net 6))
 (segment (start 135 42.69) (end 125.27 42.69) (width 0.2032) (layer "B.Cu") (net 6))
 (segment (start 104.9228 50.1172) (end 109 46.04) (width 0.1524) (layer "F.Cu") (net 9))
 (segment (start 105.96 76) (end 104.9228 74.9628) (width 0.1524) (layer "F.Cu") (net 9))
 (segment (start 104.9228 74.9628) (end 104.9228 50.1172) (width 0.1524) (layer "F.Cu") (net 9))
 (segment (start 127.0874 68.1026) (end 115.5626 68.1026) (width 0.2032) (layer "F.Cu") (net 7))
 (segment (start 115.5626 68.1026) (end 114 66.54) (width 0.2032) (layer "F.Cu") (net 7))
 (segment (start 128.19 67) (end 127.0874 68.1026) (width 0.2032) (layer "F.Cu") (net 7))
 (segment (start 128.19 64.23) (end 124.73 60.77) (width 0.2032) (layer "B.Cu") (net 7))
 (segment (start 128.19 67) (end 128.19 64.23) (width 0.2032) (layer "B.Cu") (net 7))
 (segment (start 119.5 67) (end 117.77 65.27) (width 0.2032) (layer "F.Cu") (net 1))
 (segment (start 125.5 67) (end 119.5 67) (width 0.2032) (layer "F.Cu") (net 1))
 (segment (start 117.77 65.27) (end 112.73 65.27) (width 0.2032) (layer "F.Cu") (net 1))
 (segment (start 125.5 67) (end 123.46 64.96) (width 0.2032) (layer "B.Cu") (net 1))
 (segment (start 123.46 64.96) (end 123.46 59.5) (width 0.2032) (layer "B.Cu") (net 1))
 (segment (start 106 65.12) (end 108.3726 67.4926) (width 0.2032) (layer "B.Cu") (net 2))
 (segment (start 117.3874 67.4926) (end 117.88 67) (width 0.2032) (layer "B.Cu") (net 2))
 (segment (start 108.3726 67.4926) (end 117.3874 67.4926) (width 0.2032) (layer "B.Cu") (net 2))
 (segment (start 125.0728 58.5728) (end 123.075941 58.5728) (width 0.1524) (layer "B.Cu") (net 8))
 (segment (start 119.4753 76.7772) (end 109.2772 76.7772) (width 0.1524) (layer "B.Cu") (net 8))
 (segment (start 123.075941 58.5728) (end 119.7772 61.871541) (width 0.1524) (layer "B.Cu") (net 8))
 (segment (start 109.2772 76.7772) (end 108.5 76) (width 0.1524) (layer "B.Cu") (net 8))
 (segment (start 126 59.5) (end 125.0728 58.5728) (width 0.1524) (layer "B.Cu") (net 8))
 (segment (start 119.7772 61.871541) (end 119.7772 76.4753) (width 0.1524) (layer "B.Cu") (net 8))
 (segment (start 119.7772 76.4753) (end 119.4753 76.7772) (width 0.1524) (layer "B.Cu") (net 8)))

